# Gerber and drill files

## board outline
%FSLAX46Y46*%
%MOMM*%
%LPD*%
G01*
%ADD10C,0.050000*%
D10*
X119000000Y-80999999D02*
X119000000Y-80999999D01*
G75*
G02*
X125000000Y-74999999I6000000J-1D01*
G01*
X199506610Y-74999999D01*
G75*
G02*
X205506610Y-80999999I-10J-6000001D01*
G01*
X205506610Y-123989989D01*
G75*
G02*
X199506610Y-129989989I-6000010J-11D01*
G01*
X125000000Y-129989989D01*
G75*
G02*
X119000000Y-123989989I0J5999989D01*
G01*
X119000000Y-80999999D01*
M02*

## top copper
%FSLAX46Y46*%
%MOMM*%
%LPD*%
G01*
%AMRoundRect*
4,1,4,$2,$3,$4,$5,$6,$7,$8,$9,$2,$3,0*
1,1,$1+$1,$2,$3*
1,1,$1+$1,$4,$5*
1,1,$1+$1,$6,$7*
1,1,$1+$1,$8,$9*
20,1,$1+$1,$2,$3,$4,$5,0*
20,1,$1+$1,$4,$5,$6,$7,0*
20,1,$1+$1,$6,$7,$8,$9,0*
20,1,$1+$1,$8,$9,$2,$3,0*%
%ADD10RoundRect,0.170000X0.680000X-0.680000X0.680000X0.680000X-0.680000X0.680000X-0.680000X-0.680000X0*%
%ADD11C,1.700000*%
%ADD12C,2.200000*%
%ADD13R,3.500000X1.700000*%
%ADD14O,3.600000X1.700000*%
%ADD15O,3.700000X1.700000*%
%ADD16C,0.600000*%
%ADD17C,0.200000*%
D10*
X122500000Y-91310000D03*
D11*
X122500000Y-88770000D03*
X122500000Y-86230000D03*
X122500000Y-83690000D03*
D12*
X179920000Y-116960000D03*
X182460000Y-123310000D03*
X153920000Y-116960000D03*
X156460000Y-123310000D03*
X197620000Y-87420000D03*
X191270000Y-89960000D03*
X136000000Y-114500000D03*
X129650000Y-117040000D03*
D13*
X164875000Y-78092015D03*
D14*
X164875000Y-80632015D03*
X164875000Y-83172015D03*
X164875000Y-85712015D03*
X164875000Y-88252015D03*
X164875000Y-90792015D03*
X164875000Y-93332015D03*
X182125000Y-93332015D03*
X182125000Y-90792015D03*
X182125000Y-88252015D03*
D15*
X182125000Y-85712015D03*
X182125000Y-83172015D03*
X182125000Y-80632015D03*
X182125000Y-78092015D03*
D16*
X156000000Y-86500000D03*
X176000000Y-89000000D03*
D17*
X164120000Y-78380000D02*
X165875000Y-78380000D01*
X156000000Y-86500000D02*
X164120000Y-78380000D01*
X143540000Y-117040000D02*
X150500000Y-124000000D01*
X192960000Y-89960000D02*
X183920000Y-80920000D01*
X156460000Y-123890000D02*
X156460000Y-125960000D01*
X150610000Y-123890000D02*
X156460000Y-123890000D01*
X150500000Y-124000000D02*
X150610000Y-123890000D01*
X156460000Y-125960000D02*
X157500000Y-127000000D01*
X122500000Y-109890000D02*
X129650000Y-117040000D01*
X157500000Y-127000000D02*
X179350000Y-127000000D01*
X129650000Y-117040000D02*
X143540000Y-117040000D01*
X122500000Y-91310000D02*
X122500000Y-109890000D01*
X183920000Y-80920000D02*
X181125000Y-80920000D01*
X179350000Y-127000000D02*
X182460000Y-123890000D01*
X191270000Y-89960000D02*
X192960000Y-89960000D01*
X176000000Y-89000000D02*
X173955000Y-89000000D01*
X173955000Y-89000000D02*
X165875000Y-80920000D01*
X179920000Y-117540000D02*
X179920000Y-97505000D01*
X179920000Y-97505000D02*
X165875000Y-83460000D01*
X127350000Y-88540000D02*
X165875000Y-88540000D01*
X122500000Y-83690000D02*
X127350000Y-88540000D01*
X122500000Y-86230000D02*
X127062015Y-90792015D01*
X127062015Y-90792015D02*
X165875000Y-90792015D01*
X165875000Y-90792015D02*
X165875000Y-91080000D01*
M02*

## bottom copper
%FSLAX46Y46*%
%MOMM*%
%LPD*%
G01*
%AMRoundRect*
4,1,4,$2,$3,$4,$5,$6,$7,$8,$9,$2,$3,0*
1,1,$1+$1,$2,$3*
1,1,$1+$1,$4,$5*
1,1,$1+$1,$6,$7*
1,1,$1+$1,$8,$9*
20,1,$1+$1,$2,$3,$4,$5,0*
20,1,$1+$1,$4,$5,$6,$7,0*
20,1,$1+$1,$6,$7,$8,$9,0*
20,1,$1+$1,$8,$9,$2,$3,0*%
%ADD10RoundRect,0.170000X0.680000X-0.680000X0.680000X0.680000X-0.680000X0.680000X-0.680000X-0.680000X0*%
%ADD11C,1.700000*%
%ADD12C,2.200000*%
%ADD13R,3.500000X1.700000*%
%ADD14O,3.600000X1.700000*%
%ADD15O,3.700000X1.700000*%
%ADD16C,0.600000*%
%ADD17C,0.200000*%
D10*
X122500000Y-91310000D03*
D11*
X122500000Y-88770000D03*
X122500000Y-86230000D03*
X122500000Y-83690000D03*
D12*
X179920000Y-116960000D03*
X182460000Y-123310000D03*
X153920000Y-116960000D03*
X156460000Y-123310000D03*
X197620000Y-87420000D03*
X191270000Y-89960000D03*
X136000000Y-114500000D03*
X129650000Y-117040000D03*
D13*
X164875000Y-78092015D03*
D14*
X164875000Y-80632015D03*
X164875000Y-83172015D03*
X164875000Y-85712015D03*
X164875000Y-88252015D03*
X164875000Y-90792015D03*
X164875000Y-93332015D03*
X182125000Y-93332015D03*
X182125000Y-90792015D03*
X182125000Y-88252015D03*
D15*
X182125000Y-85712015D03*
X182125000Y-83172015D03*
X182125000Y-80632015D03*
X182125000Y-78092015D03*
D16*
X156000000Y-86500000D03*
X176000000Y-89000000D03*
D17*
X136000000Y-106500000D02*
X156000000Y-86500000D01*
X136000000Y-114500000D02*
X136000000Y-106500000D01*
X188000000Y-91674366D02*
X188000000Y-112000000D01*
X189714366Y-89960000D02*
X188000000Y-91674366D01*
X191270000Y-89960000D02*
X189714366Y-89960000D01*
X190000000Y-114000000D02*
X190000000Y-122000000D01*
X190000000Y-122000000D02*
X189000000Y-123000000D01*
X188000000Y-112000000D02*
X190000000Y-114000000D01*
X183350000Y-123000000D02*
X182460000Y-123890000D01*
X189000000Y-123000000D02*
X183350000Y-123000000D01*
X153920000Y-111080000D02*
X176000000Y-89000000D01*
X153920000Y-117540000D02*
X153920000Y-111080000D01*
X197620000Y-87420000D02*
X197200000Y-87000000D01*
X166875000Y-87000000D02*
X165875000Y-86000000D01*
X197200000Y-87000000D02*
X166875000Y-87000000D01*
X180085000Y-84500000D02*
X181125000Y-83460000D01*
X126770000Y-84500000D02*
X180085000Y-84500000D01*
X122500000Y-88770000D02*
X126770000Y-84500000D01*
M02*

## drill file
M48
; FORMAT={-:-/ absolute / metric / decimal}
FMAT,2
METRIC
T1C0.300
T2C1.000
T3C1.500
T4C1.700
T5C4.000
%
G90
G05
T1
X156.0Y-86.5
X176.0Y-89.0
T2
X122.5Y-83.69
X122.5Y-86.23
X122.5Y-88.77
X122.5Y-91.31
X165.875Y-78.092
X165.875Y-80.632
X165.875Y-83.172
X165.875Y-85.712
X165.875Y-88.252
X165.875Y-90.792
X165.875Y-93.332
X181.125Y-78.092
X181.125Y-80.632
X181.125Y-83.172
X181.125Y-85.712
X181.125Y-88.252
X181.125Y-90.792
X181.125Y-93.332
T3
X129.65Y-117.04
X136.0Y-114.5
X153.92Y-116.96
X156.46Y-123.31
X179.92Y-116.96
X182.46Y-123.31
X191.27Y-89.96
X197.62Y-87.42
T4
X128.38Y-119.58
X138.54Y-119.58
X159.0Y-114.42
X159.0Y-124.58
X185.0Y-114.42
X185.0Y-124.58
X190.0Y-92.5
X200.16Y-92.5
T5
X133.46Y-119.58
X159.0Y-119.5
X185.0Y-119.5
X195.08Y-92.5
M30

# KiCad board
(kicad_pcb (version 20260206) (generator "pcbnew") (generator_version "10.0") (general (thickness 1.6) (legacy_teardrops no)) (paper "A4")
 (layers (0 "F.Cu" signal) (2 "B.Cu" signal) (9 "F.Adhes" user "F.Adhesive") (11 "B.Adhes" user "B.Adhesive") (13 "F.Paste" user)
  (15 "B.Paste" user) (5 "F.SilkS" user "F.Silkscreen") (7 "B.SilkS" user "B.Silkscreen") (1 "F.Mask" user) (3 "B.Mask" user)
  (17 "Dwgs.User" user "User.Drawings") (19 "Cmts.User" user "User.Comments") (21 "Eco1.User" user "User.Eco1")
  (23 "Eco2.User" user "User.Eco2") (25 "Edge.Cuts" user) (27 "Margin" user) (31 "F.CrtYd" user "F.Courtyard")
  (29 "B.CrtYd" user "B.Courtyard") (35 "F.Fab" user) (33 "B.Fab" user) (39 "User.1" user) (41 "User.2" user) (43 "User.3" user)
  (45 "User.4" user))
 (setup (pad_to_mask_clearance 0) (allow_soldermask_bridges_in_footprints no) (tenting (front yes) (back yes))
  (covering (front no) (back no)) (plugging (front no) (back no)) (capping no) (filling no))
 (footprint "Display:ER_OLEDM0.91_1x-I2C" (layer "F.Cu") (at 122.5 91.31 90)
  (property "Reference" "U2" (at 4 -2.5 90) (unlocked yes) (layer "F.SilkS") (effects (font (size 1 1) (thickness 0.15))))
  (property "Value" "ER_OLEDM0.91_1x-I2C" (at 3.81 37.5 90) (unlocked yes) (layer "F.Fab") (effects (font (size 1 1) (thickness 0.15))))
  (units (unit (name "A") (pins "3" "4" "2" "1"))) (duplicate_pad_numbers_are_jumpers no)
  (pad "1" thru_hole roundrect (at 0 0 90) (size 1.7 1.7) (drill 1) (layers "*.Cu" "*.Mask") (remove_unused_layers no)
   (roundrect_rratio 0.1) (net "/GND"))
  (pad "2" thru_hole circle (at 2.54 0 90) (size 1.7 1.7) (drill 1) (layers "*.Cu" "*.Mask") (remove_unused_layers no) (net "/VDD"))
  (pad "3" thru_hole circle (at 5.08 0 90) (size 1.7 1.7) (drill 1) (layers "*.Cu" "*.Mask") (remove_unused_layers no)
   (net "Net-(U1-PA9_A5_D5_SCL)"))
  (pad "4" thru_hole circle (at 7.62 0 90) (size 1.7 1.7) (drill 1) (layers "*.Cu" "*.Mask") (remove_unused_layers no)
   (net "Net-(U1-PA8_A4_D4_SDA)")))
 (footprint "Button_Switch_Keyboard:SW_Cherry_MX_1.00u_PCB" (layer "F.Cu") (at 179.92 116.96 90)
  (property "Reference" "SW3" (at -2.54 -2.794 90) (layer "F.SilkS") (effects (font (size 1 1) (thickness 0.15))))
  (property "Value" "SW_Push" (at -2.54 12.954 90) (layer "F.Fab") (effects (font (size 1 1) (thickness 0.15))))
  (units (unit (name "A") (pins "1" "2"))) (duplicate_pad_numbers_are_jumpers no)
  (pad "" np_thru_hole circle (at -7.62 5.08 90) (size 1.7 1.7) (drill 1.7) (layers "*.Cu" "*.Mask"))
  (pad "" np_thru_hole circle (at -2.54 5.08 90) (size 4 4) (drill 4) (layers "*.Cu" "*.Mask"))
  (pad "" np_thru_hole circle (at 2.54 5.08 90) (size 1.7 1.7) (drill 1.7) (layers "*.Cu" "*.Mask"))
  (pad "1" thru_hole circle (at 0 0 90) (size 2.2 2.2) (drill 1.5) (layers "*.Cu" "*.Mask") (remove_unused_layers no)
   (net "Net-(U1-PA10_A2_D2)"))
  (pad "2" thru_hole circle (at -6.35 2.54 90) (size 2.2 2.2) (drill 1.5) (layers "*.Cu" "*.Mask") (remove_unused_layers no) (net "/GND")))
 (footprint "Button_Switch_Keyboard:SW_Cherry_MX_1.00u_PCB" (layer "F.Cu") (at 153.92 116.96 90)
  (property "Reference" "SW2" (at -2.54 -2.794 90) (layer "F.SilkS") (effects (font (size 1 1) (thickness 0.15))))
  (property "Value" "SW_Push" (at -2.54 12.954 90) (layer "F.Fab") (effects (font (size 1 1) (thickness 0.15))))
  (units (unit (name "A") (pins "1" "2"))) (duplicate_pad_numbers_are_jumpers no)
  (pad "" np_thru_hole circle (at -7.62 5.08 90) (size 1.7 1.7) (drill 1.7) (layers "*.Cu" "*.Mask"))
  (pad "" np_thru_hole circle (at -2.54 5.08 90) (size 4 4) (drill 4) (layers "*.Cu" "*.Mask"))
  (pad "" np_thru_hole circle (at 2.54 5.08 90) (size 1.7 1.7) (drill 1.7) (layers "*.Cu" "*.Mask"))
  (pad "1" thru_hole circle (at 0 0 90) (size 2.2 2.2) (drill 1.5) (layers "*.Cu" "*.Mask") (remove_unused_layers no)
   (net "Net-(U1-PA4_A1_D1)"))
  (pad "2" thru_hole circle (at -6.35 2.54 90) (size 2.2 2.2) (drill 1.5) (layers "*.Cu" "*.Mask") (remove_unused_layers no) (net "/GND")))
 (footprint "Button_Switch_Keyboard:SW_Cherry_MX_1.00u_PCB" (layer "F.Cu") (at 197.62 87.42)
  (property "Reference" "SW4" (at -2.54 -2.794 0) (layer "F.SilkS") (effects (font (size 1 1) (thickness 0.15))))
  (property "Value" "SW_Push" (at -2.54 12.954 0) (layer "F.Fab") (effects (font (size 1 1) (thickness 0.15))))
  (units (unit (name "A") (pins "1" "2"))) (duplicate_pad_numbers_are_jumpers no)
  (pad "" np_thru_hole circle (at -7.62 5.08) (size 1.7 1.7) (drill 1.7) (layers "*.Cu" "*.Mask"))
  (pad "" np_thru_hole circle (at -2.54 5.08) (size 4 4) (drill 4) (layers "*.Cu" "*.Mask"))
  (pad "" np_thru_hole circle (at 2.54 5.08) (size 1.7 1.7) (drill 1.7) (layers "*.Cu" "*.Mask"))
  (pad "1" thru_hole circle (at 0 0) (size 2.2 2.2) (drill 1.5) (layers "*.Cu" "*.Mask") (remove_unused_layers no)
   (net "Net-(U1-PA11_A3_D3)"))
  (pad "2" thru_hole circle (at -6.35 2.54) (size 2.2 2.2) (drill 1.5) (layers "*.Cu" "*.Mask") (remove_unused_layers no) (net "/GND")))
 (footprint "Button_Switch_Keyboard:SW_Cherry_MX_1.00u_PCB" (layer "F.Cu") (at 136 114.5)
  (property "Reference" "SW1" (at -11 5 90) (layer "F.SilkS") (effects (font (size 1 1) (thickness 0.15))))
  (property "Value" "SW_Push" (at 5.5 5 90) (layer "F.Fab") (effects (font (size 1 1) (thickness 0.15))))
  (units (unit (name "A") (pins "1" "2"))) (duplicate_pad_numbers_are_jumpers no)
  (pad "" np_thru_hole circle (at -7.62 5.08) (size 1.7 1.7) (drill 1.7) (layers "*.Cu" "*.Mask"))
  (pad "" np_thru_hole circle (at -2.54 5.08) (size 4 4) (drill 4) (layers "*.Cu" "*.Mask"))
  (pad "" np_thru_hole circle (at 2.54 5.08) (size 1.7 1.7) (drill 1.7) (layers "*.Cu" "*.Mask"))
  (pad "1" thru_hole circle (at 0 0) (size 2.2 2.2) (drill 1.5) (layers "*.Cu" "*.Mask") (remove_unused_layers no)
   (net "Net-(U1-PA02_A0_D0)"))
  (pad "2" thru_hole circle (at -6.35 2.54) (size 2.2 2.2) (drill 1.5) (layers "*.Cu" "*.Mask") (remove_unused_layers no) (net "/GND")))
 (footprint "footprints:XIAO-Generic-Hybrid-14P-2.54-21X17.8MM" (layer "F.Cu") (at 173.5 85.712015)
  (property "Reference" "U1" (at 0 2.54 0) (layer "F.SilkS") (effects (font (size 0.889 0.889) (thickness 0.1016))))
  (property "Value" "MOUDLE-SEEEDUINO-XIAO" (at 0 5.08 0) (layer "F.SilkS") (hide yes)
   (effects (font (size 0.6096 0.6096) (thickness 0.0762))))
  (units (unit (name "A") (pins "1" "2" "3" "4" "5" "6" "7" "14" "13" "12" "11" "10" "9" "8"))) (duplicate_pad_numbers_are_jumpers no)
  (pad "1" thru_hole rect (at -7.625 -7.62) (size 3.5 1.7) (drill 1 (offset -1 0)) (layers "*.Cu" "*.Mask") (remove_unused_layers no)
   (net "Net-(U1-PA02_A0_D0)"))
  (pad "2" thru_hole oval (at -7.625 -5.08) (size 3.6 1.7) (drill 1 (offset -1 0)) (layers "*.Cu" "*.Mask") (remove_unused_layers no)
   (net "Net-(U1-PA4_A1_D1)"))
  (pad "3" thru_hole oval (at -7.625 -2.54) (size 3.6 1.7) (drill 1 (offset -1 0)) (layers "*.Cu" "*.Mask") (remove_unused_layers no)
   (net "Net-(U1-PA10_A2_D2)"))
  (pad "4" thru_hole oval (at -7.625 0) (size 3.6 1.7) (drill 1 (offset -1 0)) (layers "*.Cu" "*.Mask") (remove_unused_layers no)
   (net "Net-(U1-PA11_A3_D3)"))
  (pad "5" thru_hole oval (at -7.625 2.54) (size 3.6 1.7) (drill 1 (offset -1 0)) (layers "*.Cu" "*.Mask") (remove_unused_layers no)
   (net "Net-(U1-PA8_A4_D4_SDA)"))
  (pad "6" thru_hole oval (at -7.625 5.08 180) (size 3.6 1.7) (drill 1 (offset 1 0)) (layers "*.Cu" "*.Mask") (remove_unused_layers no)
   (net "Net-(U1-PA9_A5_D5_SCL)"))
  (pad "7" thru_hole oval (at -7.625 7.62) (size 3.6 1.7) (drill 1 (offset -1 0)) (layers "*.Cu" "*.Mask") (remove_unused_layers no)
   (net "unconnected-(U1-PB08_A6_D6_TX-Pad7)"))
  (pad "8" thru_hole oval (at 7.625 7.62) (size 3.6 1.7) (drill 1 (offset 1 0)) (layers "*.Cu" "*.Mask") (remove_unused_layers no)
   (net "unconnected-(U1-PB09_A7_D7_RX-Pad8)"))
  (pad "9" thru_hole oval (at 7.625 5.08) (size 3.6 1.7) (drill 1 (offset 1 0)) (layers "*.Cu" "*.Mask") (remove_unused_layers no)
   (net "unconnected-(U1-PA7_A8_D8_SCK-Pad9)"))
  (pad "10" thru_hole oval (at 7.625 2.54) (size 3.6 1.7) (drill 1 (offset 1 0)) (layers "*.Cu" "*.Mask") (remove_unused_layers no)
   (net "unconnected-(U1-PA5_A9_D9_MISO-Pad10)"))
  (pad "11" thru_hole oval (at 7.625 0) (size 3.7 1.7) (drill 1 (offset 1 0)) (layers "*.Cu" "*.Mask") (remove_unused_layers no)
   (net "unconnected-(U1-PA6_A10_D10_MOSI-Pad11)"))
  (pad "12" thru_hole oval (at 7.625 -2.54) (size 3.7 1.7) (drill 1 (offset 1 0)) (layers "*.Cu" "*.Mask") (remove_unused_layers no)
   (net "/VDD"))
  (pad "13" thru_hole oval (at 7.625 -5.08) (size 3.7 1.7) (drill 1 (offset 1 0)) (layers "*.Cu" "*.Mask") (remove_unused_layers no)
   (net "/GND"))
  (pad "14" thru_hole oval (at 7.625 -7.62) (size 3.7 1.7) (drill 1 (offset 1 0)) (layers "*.Cu" "*.Mask") (remove_unused_layers no)
   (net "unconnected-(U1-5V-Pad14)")))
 (gr_rect (start 119 74.999999) (end 205.50661 129.989989) (radius 6) (stroke (width 0.05) (type default)) (fill no) (layer "Edge.Cuts"))
 (segment (start 164.12 78.38) (end 165.875 78.38) (width 0.2) (layer "F.Cu") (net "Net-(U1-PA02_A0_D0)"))
 (segment (start 156 86.5) (end 164.12 78.38) (width 0.2) (layer "F.Cu") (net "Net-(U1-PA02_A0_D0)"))
 (via (at 156 86.5) (size 0.6) (drill 0.3) (layers "F.Cu" "B.Cu") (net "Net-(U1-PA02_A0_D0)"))
 (segment (start 136 106.5) (end 156 86.5) (width 0.2) (layer "B.Cu") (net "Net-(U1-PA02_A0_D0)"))
 (segment (start 136 114.5) (end 136 106.5) (width 0.2) (layer "B.Cu") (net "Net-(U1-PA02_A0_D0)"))
 (segment (start 143.54 117.04) (end 150.5 124) (width 0.2) (layer "F.Cu") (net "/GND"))
 (segment (start 192.96 89.96) (end 183.92 80.92) (width 0.2) (layer "F.Cu") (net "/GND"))
 (segment (start 156.46 123.89) (end 156.46 125.96) (width 0.2) (layer "F.Cu") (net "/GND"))
 (segment (start 150.61 123.89) (end 156.46 123.89) (width 0.2) (layer "F.Cu") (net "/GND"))
 (segment (start 150.5 124) (end 150.61 123.89) (width 0.2) (layer "F.Cu") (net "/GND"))
 (segment (start 156.46 125.96) (end 157.5 127) (width 0.2) (layer "F.Cu") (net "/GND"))
 (segment (start 122.5 109.89) (end 129.65 117.04) (width 0.2) (layer "F.Cu") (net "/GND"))
 (segment (start 157.5 127) (end 179.35 127) (width 0.2) (layer "F.Cu") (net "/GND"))
 (segment (start 129.65 117.04) (end 143.54 117.04) (width 0.2) (layer "F.Cu") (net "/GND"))
 (segment (start 122.5 91.31) (end 122.5 109.89) (width 0.2) (layer "F.Cu") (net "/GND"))
 (segment (start 183.92 80.92) (end 181.125 80.92) (width 0.2) (layer "F.Cu") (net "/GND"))
 (segment (start 179.35 127) (end 182.46 123.89) (width 0.2) (layer "F.Cu") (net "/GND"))
 (segment (start 191.27 89.96) (end 192.96 89.96) (width 0.2) (layer "F.Cu") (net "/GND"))
 (segment (start 188 91.674366) (end 188 112) (width 0.2) (layer "B.Cu") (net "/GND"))
 (segment (start 189.714366 89.96) (end 188 91.674366) (width 0.2) (layer "B.Cu") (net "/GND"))
 (segment (start 191.27 89.96) (end 189.714366 89.96) (width 0.2) (layer "B.Cu") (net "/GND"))
 (segment (start 190 114) (end 190 122) (width 0.2) (layer "B.Cu") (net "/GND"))
 (segment (start 190 122) (end 189 123) (width 0.2) (layer "B.Cu") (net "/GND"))
 (segment (start 188 112) (end 190 114) (width 0.2) (layer "B.Cu") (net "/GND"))
 (segment (start 183.35 123) (end 182.46 123.89) (width 0.2) (layer "B.Cu") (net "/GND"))
 (segment (start 189 123) (end 183.35 123) (width 0.2) (layer "B.Cu") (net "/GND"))
 (segment (start 176 89) (end 173.955 89) (width 0.2) (layer "F.Cu") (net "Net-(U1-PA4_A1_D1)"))
 (segment (start 173.955 89) (end 165.875 80.92) (width 0.2) (layer "F.Cu") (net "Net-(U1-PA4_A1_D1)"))
 (via (at 176 89) (size 0.6) (drill 0.3) (layers "F.Cu" "B.Cu") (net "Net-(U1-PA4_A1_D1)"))
 (segment (start 153.92 111.08) (end 176 89) (width 0.2) (layer "B.Cu") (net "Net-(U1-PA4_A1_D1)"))
 (segment (start 153.92 117.54) (end 153.92 111.08) (width 0.2) (layer "B.Cu") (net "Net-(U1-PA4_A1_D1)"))
 (segment (start 179.92 117.54) (end 179.92 97.505) (width 0.2) (layer "F.Cu") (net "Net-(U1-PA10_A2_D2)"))
 (segment (start 179.92 97.505) (end 165.875 83.46) (width 0.2) (layer "F.Cu") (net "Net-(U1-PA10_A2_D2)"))
 (segment (start 197.62 87.42) (end 197.2 87) (width 0.2) (layer "B.Cu") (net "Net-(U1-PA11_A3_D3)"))
 (segment (start 166.875 87) (end 165.875 86) (width 0.2) (layer "B.Cu") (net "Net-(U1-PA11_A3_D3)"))
 (segment (start 197.2 87) (end 166.875 87) (width 0.2) (layer "B.Cu") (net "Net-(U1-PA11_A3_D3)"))
 (segment (start 127.35 88.54) (end 165.875 88.54) (width 0.2) (layer "F.Cu") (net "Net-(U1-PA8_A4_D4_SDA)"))
 (segment (start 122.5 83.69) (end 127.35 88.54) (width 0.2) (layer "F.Cu") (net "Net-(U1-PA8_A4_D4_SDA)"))
 (segment (start 122.5 86.23) (end 127.062015 90.792015) (width 0.2) (layer "F.Cu") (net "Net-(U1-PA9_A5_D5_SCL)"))
 (segment (start 127.062015 90.792015) (end 165.875 90.792015) (width 0.2) (layer "F.Cu") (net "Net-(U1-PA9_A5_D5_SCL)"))
 (segment (start 165.875 90.792015) (end 165.875 91.08) (width 0.2) (layer "F.Cu") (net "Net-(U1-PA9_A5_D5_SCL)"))
 (segment (start 180.085 84.5) (end 181.125 83.46) (width 0.2) (layer "B.Cu") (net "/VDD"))
 (segment (start 126.77 84.5) (end 180.085 84.5) (width 0.2) (layer "B.Cu") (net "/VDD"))
 (segment (start 122.5 88.77) (end 126.77 84.5) (width 0.2) (layer "B.Cu") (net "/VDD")))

